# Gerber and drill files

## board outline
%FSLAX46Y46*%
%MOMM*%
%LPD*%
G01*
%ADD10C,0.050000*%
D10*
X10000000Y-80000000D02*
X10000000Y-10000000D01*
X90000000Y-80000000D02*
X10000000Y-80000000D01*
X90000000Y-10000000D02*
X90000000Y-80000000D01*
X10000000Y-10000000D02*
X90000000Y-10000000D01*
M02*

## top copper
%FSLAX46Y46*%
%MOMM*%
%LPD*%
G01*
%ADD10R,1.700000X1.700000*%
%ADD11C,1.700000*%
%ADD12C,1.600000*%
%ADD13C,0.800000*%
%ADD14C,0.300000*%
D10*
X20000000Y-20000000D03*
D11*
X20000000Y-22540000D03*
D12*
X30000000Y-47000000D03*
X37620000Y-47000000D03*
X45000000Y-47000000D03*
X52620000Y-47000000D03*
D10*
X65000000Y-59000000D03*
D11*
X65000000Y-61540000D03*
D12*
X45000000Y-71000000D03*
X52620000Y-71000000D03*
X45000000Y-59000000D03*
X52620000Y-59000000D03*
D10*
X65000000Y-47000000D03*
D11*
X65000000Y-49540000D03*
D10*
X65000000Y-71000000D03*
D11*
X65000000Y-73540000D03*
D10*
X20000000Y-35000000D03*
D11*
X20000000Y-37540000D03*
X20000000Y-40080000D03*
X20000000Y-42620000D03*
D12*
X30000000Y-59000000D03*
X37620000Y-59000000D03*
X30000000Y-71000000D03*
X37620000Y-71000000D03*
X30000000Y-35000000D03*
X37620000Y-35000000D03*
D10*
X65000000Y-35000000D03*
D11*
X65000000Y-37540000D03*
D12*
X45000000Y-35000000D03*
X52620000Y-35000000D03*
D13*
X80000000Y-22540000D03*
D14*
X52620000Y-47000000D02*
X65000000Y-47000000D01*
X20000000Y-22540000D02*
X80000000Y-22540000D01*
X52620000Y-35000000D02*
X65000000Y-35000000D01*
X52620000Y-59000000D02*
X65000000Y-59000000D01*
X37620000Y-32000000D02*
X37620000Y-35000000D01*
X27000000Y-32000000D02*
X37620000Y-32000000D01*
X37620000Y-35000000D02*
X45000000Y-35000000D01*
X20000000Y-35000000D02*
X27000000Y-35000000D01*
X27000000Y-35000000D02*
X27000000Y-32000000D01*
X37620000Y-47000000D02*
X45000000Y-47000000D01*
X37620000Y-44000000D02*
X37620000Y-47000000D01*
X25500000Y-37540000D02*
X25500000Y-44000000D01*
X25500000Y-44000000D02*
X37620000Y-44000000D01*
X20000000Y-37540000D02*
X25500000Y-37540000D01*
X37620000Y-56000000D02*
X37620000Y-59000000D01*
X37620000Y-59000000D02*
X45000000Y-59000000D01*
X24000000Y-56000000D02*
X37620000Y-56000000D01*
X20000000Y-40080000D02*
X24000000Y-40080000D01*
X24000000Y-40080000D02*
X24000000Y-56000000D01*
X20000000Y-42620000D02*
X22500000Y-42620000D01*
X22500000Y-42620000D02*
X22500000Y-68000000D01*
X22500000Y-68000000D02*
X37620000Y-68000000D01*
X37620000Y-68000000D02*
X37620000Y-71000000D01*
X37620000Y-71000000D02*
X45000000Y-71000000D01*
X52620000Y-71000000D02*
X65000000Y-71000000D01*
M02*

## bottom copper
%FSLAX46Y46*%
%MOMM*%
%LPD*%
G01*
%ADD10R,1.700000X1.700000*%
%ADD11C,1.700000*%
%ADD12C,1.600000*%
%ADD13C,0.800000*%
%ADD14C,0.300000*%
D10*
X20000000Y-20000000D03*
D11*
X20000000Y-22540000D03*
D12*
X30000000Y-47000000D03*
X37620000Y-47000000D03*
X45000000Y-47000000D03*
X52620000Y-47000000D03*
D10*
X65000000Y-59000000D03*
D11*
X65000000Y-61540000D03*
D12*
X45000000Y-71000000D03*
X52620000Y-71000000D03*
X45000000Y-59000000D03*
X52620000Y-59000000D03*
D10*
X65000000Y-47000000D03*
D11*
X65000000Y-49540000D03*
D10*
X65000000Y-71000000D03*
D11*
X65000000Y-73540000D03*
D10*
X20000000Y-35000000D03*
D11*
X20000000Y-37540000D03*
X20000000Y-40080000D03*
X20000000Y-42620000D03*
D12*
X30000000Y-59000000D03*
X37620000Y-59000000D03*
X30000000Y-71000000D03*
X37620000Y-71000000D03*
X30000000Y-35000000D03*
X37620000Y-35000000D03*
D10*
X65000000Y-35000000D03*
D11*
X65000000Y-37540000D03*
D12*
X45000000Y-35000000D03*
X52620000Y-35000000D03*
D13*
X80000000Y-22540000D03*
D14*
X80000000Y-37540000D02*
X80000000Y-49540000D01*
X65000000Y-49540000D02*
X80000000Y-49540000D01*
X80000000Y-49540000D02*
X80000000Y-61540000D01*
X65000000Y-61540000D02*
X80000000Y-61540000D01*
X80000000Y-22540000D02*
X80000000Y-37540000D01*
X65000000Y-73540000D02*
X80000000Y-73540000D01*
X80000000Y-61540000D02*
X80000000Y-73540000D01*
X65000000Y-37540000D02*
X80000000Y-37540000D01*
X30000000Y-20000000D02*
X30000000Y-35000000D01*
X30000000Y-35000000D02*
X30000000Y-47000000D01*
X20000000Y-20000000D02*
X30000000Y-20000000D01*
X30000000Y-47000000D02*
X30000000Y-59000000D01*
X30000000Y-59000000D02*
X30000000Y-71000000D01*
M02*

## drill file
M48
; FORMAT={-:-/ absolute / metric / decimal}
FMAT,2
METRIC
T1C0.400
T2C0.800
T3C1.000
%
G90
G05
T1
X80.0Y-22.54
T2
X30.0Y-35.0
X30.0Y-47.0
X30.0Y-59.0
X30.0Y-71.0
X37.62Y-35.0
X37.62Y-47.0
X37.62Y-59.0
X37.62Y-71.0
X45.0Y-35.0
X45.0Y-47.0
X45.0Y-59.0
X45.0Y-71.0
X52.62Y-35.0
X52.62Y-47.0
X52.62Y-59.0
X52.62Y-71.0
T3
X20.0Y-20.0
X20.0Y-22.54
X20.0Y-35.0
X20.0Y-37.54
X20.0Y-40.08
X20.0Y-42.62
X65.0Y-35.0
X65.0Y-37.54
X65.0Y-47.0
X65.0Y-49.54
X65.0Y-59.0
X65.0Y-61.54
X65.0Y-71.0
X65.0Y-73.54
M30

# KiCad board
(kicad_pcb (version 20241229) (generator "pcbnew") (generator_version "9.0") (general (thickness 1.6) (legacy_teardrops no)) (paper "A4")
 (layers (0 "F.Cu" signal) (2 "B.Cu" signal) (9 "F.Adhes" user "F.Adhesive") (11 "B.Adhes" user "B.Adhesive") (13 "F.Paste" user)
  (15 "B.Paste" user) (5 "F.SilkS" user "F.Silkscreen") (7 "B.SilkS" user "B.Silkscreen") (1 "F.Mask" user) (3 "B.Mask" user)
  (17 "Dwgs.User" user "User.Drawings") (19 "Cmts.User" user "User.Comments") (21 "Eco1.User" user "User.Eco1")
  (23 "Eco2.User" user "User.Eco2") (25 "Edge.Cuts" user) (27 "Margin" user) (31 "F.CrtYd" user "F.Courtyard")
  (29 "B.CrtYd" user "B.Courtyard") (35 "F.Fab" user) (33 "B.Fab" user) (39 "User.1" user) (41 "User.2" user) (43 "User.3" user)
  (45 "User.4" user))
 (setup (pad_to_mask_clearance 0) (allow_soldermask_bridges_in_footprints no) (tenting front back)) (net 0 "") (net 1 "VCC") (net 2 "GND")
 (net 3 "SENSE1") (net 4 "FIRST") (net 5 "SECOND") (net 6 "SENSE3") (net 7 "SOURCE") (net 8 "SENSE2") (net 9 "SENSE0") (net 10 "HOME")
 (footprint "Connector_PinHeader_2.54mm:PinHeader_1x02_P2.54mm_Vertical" (layer "F.Cu") (at 20 20)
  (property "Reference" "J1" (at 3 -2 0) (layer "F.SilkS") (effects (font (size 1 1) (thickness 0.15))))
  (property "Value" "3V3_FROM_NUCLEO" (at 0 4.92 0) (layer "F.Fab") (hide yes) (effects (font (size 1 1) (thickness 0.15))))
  (pad "1" thru_hole rect (at 0 0) (size 1.7 1.7) (drill 1) (layers "*.Cu" "*.Mask") (remove_unused_layers no) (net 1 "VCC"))
  (pad "2" thru_hole circle (at 0 2.54) (size 1.7 1.7) (drill 1) (layers "*.Cu" "*.Mask") (remove_unused_layers no) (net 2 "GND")))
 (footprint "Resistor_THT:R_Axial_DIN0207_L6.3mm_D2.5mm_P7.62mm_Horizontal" (layer "F.Cu") (at 30 47)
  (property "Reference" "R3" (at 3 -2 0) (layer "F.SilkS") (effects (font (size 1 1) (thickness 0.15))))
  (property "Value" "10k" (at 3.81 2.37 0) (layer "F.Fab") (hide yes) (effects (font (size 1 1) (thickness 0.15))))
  (pad "1" thru_hole circle (at 0 0) (size 1.6 1.6) (drill 0.8) (layers "*.Cu" "*.Mask") (remove_unused_layers no) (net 1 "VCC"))
  (pad "2" thru_hole circle (at 7.62 0) (size 1.6 1.6) (drill 0.8) (layers "*.Cu" "*.Mask") (remove_unused_layers no) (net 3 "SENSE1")))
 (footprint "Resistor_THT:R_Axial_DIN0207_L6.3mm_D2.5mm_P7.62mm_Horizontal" (layer "F.Cu") (at 45 47)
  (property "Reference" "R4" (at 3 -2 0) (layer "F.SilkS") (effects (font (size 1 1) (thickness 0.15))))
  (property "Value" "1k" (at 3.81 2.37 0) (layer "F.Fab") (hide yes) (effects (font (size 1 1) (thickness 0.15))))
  (pad "1" thru_hole circle (at 0 0) (size 1.6 1.6) (drill 0.8) (layers "*.Cu" "*.Mask") (remove_unused_layers no) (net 3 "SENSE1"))
  (pad "2" thru_hole circle (at 7.62 0) (size 1.6 1.6) (drill 0.8) (layers "*.Cu" "*.Mask") (remove_unused_layers no) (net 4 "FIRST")))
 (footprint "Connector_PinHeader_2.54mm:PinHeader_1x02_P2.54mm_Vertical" (layer "F.Cu") (at 65 59)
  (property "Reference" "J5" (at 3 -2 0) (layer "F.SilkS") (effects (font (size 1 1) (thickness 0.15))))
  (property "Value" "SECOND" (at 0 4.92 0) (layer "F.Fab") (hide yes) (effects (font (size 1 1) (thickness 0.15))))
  (pad "1" thru_hole rect (at 0 0) (size 1.7 1.7) (drill 1) (layers "*.Cu" "*.Mask") (remove_unused_layers no) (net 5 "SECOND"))
  (pad "2" thru_hole circle (at 0 2.54) (size 1.7 1.7) (drill 1) (layers "*.Cu" "*.Mask") (remove_unused_layers no) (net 2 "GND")))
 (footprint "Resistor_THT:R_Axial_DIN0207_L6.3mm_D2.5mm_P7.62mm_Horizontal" (layer "F.Cu") (at 45 71)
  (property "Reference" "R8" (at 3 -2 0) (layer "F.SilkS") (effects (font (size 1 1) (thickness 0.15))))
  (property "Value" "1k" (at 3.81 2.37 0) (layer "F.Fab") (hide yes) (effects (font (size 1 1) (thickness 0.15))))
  (pad "1" thru_hole circle (at 0 0) (size 1.6 1.6) (drill 0.8) (layers "*.Cu" "*.Mask") (remove_unused_layers no) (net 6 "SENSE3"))
  (pad "2" thru_hole circle (at 7.62 0) (size 1.6 1.6) (drill 0.8) (layers "*.Cu" "*.Mask") (remove_unused_layers no) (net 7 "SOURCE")))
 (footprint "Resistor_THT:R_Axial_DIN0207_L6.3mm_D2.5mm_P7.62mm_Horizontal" (layer "F.Cu") (at 45 59)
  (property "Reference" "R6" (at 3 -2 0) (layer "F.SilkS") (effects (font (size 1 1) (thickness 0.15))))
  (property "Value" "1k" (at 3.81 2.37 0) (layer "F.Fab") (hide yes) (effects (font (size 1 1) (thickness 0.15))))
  (pad "1" thru_hole circle (at 0 0) (size 1.6 1.6) (drill 0.8) (layers "*.Cu" "*.Mask") (remove_unused_layers no) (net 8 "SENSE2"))
  (pad "2" thru_hole circle (at 7.62 0) (size 1.6 1.6) (drill 0.8) (layers "*.Cu" "*.Mask") (remove_unused_layers no) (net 5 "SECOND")))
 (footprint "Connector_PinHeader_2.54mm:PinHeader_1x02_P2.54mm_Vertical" (layer "F.Cu") (at 65 47)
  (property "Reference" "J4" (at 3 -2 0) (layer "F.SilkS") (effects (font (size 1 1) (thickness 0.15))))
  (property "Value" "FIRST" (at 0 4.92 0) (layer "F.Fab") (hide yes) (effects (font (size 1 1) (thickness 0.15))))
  (pad "1" thru_hole rect (at 0 0) (size 1.7 1.7) (drill 1) (layers "*.Cu" "*.Mask") (remove_unused_layers no) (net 4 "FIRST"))
  (pad "2" thru_hole circle (at 0 2.54) (size 1.7 1.7) (drill 1) (layers "*.Cu" "*.Mask") (remove_unused_layers no) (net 2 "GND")))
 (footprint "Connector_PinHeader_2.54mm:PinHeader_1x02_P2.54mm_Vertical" (layer "F.Cu") (at 65 71)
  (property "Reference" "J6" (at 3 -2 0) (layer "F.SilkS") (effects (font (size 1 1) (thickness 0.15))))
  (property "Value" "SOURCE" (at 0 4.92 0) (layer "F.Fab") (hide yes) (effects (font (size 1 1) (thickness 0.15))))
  (pad "1" thru_hole rect (at 0 0) (size 1.7 1.7) (drill 1) (layers "*.Cu" "*.Mask") (remove_unused_layers no) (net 7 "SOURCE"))
  (pad "2" thru_hole circle (at 0 2.54) (size 1.7 1.7) (drill 1) (layers "*.Cu" "*.Mask") (remove_unused_layers no) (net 2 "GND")))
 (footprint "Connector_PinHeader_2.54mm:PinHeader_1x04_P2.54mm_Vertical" (layer "F.Cu") (at 20 35)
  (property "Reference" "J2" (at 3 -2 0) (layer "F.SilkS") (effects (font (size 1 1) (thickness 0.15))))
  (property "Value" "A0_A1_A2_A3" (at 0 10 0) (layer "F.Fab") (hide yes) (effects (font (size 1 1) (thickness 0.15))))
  (pad "1" thru_hole rect (at 0 0) (size 1.7 1.7) (drill 1) (layers "*.Cu" "*.Mask") (remove_unused_layers no) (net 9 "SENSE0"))
  (pad "2" thru_hole circle (at 0 2.54) (size 1.7 1.7) (drill 1) (layers "*.Cu" "*.Mask") (remove_unused_layers no) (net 3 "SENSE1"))
  (pad "3" thru_hole circle (at 0 5.08) (size 1.7 1.7) (drill 1) (layers "*.Cu" "*.Mask") (remove_unused_layers no) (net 8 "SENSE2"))
  (pad "4" thru_hole circle (at 0 7.62) (size 1.7 1.7) (drill 1) (layers "*.Cu" "*.Mask") (remove_unused_layers no) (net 6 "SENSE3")))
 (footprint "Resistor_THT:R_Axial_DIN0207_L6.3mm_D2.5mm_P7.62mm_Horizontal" (layer "F.Cu") (at 30 59)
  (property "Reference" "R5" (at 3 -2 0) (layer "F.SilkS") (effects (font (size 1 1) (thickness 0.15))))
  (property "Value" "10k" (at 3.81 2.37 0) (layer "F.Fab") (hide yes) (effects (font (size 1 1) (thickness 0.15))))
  (pad "1" thru_hole circle (at 0 0) (size 1.6 1.6) (drill 0.8) (layers "*.Cu" "*.Mask") (remove_unused_layers no) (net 1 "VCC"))
  (pad "2" thru_hole circle (at 7.62 0) (size 1.6 1.6) (drill 0.8) (layers "*.Cu" "*.Mask") (remove_unused_layers no) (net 8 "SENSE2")))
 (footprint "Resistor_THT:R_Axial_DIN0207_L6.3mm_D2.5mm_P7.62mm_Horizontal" (layer "F.Cu") (at 30 71)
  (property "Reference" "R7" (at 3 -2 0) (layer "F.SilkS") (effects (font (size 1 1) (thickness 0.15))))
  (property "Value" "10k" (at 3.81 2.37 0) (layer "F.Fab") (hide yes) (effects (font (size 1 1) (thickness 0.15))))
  (pad "1" thru_hole circle (at 0 0) (size 1.6 1.6) (drill 0.8) (layers "*.Cu" "*.Mask") (remove_unused_layers no) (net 1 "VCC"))
  (pad "2" thru_hole circle (at 7.62 0) (size 1.6 1.6) (drill 0.8) (layers "*.Cu" "*.Mask") (remove_unused_layers no) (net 6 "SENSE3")))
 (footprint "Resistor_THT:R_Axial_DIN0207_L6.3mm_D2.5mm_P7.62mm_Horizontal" (layer "F.Cu") (at 30 35)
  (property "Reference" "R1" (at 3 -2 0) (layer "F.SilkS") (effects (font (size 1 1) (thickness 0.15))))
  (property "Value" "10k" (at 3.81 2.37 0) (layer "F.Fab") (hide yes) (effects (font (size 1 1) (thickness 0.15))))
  (pad "1" thru_hole circle (at 0 0) (size 1.6 1.6) (drill 0.8) (layers "*.Cu" "*.Mask") (remove_unused_layers no) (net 1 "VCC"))
  (pad "2" thru_hole circle (at 7.62 0) (size 1.6 1.6) (drill 0.8) (layers "*.Cu" "*.Mask") (remove_unused_layers no) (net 9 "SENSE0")))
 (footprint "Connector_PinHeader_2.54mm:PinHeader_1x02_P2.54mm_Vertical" (layer "F.Cu") (at 65 35)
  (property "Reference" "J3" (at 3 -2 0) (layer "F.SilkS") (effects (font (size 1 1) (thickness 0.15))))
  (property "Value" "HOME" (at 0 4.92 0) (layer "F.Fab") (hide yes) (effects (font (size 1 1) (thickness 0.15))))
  (pad "1" thru_hole rect (at 0 0) (size 1.7 1.7) (drill 1) (layers "*.Cu" "*.Mask") (remove_unused_layers no) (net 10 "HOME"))
  (pad "2" thru_hole circle (at 0 2.54) (size 1.7 1.7) (drill 1) (layers "*.Cu" "*.Mask") (remove_unused_layers no) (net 2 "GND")))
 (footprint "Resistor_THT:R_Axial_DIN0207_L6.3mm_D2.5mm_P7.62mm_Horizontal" (layer "F.Cu") (at 45 35)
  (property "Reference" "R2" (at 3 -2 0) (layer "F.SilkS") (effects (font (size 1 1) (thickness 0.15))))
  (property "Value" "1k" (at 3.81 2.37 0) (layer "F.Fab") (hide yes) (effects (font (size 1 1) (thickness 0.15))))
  (pad "1" thru_hole circle (at 0 0) (size 1.6 1.6) (drill 0.8) (layers "*.Cu" "*.Mask") (remove_unused_layers no) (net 9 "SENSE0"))
  (pad "2" thru_hole circle (at 7.62 0) (size 1.6 1.6) (drill 0.8) (layers "*.Cu" "*.Mask") (remove_unused_layers no) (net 10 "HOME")))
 (gr_line (start 10 80) (end 10 10) (stroke (width 0.05) (type default)) (layer "Edge.Cuts"))
 (gr_line (start 90 80) (end 10 80) (stroke (width 0.05) (type default)) (layer "Edge.Cuts"))
 (gr_line (start 90 10) (end 90 80) (stroke (width 0.05) (type default)) (layer "Edge.Cuts"))
 (gr_line (start 10 10) (end 90 10) (stroke (width 0.05) (type default)) (layer "Edge.Cuts"))
 (segment (start 52.62 47) (end 65 47) (width 0.3) (layer "F.Cu") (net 4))
 (segment (start 20 22.54) (end 80 22.54) (width 0.3) (layer "F.Cu") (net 2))
 (via (at 80 22.54) (size 0.8) (drill 0.4) (layers "F.Cu" "B.Cu") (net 2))
 (segment (start 80 37.54) (end 80 49.54) (width 0.3) (layer "B.Cu") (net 2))
 (segment (start 65 49.54) (end 80 49.54) (width 0.3) (layer "B.Cu") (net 2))
 (segment (start 80 49.54) (end 80 61.54) (width 0.3) (layer "B.Cu") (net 2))
 (segment (start 65 61.54) (end 80 61.54) (width 0.3) (layer "B.Cu") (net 2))
 (segment (start 80 22.54) (end 80 37.54) (width 0.3) (layer "B.Cu") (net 2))
 (segment (start 65 73.54) (end 80 73.54) (width 0.3) (layer "B.Cu") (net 2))
 (segment (start 80 61.54) (end 80 73.54) (width 0.3) (layer "B.Cu") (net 2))
 (segment (start 65 37.54) (end 80 37.54) (width 0.3) (layer "B.Cu") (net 2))
 (segment (start 52.62 35) (end 65 35) (width 0.3) (layer "F.Cu") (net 10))
 (segment (start 52.62 59) (end 65 59) (width 0.3) (layer "F.Cu") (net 5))
 (segment (start 37.62 32) (end 37.62 35) (width 0.3) (layer "F.Cu") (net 9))
 (segment (start 27 32) (end 37.62 32) (width 0.3) (layer "F.Cu") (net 9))
 (segment (start 37.62 35) (end 45 35) (width 0.3) (layer "F.Cu") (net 9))
 (segment (start 20 35) (end 27 35) (width 0.3) (layer "F.Cu") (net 9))
 (segment (start 27 35) (end 27 32) (width 0.3) (layer "F.Cu") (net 9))
 (segment (start 37.62 47) (end 45 47) (width 0.3) (layer "F.Cu") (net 3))
 (segment (start 37.62 44) (end 37.62 47) (width 0.3) (layer "F.Cu") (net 3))
 (segment (start 25.5 37.54) (end 25.5 44) (width 0.3) (layer "F.Cu") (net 3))
 (segment (start 25.5 44) (end 37.62 44) (width 0.3) (layer "F.Cu") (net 3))
 (segment (start 20 37.54) (end 25.5 37.54) (width 0.3) (layer "F.Cu") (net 3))
 (segment (start 37.62 56) (end 37.62 59) (width 0.3) (layer "F.Cu") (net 8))
 (segment (start 37.62 59) (end 45 59) (width 0.3) (layer "F.Cu") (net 8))
 (segment (start 24 56) (end 37.62 56) (width 0.3) (layer "F.Cu") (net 8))
 (segment (start 20 40.08) (end 24 40.08) (width 0.3) (layer "F.Cu") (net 8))
 (segment (start 24 40.08) (end 24 56) (width 0.3) (layer "F.Cu") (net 8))
 (segment (start 20 42.62) (end 22.5 42.62) (width 0.3) (layer "F.Cu") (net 6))
 (segment (start 22.5 42.62) (end 22.5 68) (width 0.3) (layer "F.Cu") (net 6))
 (segment (start 22.5 68) (end 37.62 68) (width 0.3) (layer "F.Cu") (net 6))
 (segment (start 37.62 68) (end 37.62 71) (width 0.3) (layer "F.Cu") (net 6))
 (segment (start 37.62 71) (end 45 71) (width 0.3) (layer "F.Cu") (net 6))
 (segment (start 52.62 71) (end 65 71) (width 0.3) (layer "F.Cu") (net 7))
 (segment (start 30 20) (end 30 35) (width 0.3) (layer "B.Cu") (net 1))
 (segment (start 30 35) (end 30 47) (width 0.3) (layer "B.Cu") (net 1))
 (segment (start 20 20) (end 30 20) (width 0.3) (layer "B.Cu") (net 1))
 (segment (start 30 47) (end 30 59) (width 0.3) (layer "B.Cu") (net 1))
 (segment (start 30 59) (end 30 71) (width 0.3) (layer "B.Cu") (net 1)))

